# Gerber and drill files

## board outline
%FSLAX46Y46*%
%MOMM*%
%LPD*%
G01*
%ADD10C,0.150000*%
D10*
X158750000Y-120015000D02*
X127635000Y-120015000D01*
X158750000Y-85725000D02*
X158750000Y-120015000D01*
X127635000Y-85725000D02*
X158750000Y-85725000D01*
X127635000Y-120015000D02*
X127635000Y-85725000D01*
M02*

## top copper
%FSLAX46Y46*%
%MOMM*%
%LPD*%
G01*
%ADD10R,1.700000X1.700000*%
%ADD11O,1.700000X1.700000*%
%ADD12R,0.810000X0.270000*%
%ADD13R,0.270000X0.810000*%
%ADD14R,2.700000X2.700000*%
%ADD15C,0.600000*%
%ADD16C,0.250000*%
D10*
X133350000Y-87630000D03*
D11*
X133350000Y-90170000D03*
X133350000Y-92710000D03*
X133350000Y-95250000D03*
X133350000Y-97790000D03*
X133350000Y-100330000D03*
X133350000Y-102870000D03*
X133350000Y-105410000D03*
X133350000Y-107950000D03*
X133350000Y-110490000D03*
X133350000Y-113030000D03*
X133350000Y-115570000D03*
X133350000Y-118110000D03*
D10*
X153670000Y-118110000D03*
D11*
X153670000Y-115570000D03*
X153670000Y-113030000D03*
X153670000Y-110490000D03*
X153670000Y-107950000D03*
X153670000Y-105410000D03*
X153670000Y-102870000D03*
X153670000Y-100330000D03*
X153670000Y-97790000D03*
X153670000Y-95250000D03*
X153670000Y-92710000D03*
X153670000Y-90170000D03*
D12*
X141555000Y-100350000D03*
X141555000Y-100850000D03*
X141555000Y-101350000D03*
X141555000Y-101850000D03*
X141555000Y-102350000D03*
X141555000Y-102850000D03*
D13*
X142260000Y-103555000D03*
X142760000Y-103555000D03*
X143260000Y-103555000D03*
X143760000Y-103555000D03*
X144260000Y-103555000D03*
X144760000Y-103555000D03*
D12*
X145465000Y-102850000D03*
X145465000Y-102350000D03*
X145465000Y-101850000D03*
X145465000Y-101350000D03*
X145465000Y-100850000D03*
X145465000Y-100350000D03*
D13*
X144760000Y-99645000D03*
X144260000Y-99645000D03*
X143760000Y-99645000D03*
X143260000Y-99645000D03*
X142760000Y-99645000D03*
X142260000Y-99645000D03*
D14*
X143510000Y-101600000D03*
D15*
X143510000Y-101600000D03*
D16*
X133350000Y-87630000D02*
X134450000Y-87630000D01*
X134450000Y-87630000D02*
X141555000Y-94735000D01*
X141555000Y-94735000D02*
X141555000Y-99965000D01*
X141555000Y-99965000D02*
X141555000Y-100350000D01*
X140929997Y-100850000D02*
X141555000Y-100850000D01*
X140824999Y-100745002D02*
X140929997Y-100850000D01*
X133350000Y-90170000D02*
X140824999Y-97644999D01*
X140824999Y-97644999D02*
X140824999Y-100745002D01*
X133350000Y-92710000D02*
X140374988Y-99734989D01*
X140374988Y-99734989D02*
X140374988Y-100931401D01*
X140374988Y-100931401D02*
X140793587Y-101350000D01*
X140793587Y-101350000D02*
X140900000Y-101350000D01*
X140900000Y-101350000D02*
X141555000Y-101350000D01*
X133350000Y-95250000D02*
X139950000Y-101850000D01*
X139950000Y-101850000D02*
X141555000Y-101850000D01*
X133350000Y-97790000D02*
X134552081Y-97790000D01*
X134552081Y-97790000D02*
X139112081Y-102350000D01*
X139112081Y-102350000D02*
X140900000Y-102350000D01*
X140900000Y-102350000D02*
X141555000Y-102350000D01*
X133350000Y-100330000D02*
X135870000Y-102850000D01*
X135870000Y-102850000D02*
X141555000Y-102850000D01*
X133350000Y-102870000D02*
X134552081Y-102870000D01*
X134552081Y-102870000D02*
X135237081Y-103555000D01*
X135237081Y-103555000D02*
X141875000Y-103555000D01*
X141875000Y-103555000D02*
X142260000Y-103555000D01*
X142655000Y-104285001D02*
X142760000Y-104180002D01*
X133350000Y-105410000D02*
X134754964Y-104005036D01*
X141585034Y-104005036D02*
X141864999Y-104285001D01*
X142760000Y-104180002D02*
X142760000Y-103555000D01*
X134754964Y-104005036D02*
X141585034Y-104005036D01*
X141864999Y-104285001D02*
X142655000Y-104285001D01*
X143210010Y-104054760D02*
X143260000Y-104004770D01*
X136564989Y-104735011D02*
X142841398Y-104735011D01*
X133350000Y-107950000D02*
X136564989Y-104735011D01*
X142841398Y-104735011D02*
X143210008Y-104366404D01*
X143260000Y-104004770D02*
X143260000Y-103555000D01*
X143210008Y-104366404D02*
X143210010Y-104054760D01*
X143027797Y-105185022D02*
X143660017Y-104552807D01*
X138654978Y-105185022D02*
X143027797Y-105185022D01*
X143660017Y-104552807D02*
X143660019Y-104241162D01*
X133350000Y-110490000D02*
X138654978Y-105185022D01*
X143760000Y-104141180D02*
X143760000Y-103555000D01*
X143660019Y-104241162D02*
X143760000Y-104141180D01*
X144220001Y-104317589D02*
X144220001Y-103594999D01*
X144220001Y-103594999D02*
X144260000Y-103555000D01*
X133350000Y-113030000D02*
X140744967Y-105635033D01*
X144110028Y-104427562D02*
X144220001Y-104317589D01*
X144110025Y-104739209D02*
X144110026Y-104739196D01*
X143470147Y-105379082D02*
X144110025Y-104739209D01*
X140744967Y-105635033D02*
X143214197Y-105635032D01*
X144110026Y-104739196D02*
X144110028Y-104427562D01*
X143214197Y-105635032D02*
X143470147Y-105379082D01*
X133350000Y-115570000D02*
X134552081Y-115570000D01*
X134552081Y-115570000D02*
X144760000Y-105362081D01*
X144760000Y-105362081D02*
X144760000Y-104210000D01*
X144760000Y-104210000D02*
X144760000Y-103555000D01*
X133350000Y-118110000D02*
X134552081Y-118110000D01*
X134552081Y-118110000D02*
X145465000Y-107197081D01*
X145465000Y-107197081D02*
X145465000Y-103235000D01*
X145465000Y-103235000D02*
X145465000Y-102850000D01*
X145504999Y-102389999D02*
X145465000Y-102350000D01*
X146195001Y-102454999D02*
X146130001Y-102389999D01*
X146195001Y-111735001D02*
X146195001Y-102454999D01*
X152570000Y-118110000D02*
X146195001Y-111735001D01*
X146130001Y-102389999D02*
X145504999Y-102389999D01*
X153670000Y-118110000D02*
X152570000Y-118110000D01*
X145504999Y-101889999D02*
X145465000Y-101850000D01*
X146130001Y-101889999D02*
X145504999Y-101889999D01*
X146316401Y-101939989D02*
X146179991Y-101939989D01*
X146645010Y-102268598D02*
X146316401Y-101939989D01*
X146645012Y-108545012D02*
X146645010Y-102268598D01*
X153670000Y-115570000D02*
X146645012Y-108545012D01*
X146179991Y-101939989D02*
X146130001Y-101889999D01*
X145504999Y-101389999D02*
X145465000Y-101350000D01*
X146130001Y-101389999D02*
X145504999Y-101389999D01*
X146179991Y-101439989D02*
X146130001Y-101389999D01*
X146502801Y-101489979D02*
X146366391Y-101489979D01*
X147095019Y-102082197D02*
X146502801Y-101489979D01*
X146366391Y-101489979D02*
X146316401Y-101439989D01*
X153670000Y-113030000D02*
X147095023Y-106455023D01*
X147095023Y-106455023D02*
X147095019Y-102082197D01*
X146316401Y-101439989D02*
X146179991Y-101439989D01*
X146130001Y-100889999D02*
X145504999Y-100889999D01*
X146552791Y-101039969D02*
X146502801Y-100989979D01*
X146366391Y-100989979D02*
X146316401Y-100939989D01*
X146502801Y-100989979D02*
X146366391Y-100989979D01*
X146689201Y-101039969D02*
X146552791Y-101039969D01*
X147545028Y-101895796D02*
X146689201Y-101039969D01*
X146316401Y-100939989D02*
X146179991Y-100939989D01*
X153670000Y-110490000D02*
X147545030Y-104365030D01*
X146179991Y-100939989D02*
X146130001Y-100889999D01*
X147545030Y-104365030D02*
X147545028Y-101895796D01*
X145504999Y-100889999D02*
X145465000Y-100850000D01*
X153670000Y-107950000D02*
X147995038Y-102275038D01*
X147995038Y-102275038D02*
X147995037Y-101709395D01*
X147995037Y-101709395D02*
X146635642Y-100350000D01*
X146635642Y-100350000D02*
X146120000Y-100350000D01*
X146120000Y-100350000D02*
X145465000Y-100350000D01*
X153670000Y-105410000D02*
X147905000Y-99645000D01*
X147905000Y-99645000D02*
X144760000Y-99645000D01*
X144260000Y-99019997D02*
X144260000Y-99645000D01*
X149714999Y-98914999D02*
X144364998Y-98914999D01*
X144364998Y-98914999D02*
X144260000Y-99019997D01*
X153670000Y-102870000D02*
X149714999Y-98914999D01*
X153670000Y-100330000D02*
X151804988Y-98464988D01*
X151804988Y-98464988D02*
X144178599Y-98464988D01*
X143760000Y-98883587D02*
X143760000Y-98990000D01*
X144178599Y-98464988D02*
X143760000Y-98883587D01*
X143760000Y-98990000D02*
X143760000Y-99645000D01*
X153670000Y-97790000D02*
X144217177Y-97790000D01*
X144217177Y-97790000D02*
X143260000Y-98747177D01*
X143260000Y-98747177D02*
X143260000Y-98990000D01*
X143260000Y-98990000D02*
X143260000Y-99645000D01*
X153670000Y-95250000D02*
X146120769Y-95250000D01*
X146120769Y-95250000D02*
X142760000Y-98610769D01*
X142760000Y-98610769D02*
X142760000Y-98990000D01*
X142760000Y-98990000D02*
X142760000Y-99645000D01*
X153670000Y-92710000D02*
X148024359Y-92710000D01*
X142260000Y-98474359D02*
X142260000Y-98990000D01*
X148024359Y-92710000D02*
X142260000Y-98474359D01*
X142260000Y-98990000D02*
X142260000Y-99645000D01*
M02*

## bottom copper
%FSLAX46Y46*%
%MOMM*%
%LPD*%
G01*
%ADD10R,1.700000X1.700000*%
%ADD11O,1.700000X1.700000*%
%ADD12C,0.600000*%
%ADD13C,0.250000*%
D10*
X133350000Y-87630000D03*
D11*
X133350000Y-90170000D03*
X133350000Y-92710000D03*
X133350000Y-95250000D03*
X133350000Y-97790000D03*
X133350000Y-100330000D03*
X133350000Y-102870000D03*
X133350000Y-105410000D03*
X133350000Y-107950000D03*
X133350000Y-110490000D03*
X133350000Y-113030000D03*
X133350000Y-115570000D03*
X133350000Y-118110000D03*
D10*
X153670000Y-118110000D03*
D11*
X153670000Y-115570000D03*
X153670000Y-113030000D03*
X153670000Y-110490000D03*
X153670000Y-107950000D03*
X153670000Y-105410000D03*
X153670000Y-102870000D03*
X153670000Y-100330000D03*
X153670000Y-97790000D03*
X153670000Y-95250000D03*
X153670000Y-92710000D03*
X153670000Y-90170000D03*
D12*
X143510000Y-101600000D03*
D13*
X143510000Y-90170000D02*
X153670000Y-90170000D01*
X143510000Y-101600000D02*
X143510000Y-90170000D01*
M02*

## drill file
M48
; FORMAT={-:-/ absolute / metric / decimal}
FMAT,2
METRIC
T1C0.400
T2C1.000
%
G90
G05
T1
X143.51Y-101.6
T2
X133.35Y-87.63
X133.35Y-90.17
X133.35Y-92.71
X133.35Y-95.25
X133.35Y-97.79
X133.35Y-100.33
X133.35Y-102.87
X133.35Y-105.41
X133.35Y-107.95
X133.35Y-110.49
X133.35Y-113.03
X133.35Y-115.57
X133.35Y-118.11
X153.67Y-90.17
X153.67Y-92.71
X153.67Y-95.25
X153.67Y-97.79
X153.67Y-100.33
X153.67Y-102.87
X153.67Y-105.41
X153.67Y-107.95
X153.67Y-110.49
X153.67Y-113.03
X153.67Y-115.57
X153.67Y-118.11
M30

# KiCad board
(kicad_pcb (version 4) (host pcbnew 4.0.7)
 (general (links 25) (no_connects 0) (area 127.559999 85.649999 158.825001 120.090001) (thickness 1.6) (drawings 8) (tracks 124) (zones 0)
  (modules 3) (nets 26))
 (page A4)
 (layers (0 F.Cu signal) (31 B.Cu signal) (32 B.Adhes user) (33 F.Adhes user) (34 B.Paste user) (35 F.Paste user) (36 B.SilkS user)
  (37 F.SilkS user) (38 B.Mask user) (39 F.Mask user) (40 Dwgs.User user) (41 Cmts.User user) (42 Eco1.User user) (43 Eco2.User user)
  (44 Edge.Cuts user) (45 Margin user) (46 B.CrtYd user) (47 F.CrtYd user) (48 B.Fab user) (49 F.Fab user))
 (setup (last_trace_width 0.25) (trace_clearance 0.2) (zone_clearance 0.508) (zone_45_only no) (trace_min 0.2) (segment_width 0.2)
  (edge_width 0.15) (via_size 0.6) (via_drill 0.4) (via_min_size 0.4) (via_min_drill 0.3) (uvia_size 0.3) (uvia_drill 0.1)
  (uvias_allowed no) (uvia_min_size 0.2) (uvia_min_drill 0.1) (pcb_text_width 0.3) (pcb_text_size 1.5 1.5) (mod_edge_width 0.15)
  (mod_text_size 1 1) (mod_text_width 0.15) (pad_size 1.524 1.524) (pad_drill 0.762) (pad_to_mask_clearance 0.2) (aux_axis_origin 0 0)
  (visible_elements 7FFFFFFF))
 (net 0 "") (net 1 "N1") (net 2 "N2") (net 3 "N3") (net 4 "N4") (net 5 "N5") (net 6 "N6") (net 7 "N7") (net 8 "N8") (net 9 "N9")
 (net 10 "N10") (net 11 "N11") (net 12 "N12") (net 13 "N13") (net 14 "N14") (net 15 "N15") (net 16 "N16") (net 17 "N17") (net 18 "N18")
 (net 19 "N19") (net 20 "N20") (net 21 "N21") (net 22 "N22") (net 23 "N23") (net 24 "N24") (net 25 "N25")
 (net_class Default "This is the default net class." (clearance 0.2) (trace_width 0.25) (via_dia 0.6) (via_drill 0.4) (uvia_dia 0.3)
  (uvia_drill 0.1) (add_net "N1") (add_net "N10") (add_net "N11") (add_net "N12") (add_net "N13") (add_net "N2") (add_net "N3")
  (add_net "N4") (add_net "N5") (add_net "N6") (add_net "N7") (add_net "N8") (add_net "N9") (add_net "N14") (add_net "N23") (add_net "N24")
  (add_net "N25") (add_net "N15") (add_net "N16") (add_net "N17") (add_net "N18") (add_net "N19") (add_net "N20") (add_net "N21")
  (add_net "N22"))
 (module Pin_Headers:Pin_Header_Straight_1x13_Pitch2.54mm (layer F.Cu) (at 133.35 87.63)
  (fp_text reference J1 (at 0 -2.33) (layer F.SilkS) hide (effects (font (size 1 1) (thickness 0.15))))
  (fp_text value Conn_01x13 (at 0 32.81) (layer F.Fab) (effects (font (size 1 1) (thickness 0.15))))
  (pad 1 thru_hole rect (at 0 0) (size 1.7 1.7) (drill 1) (layers *.Cu *.Mask) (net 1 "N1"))
  (pad 2 thru_hole oval (at 0 2.54) (size 1.7 1.7) (drill 1) (layers *.Cu *.Mask) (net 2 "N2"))
  (pad 3 thru_hole oval (at 0 5.08) (size 1.7 1.7) (drill 1) (layers *.Cu *.Mask) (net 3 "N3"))
  (pad 4 thru_hole oval (at 0 7.62) (size 1.7 1.7) (drill 1) (layers *.Cu *.Mask) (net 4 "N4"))
  (pad 5 thru_hole oval (at 0 10.16) (size 1.7 1.7) (drill 1) (layers *.Cu *.Mask) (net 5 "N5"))
  (pad 6 thru_hole oval (at 0 12.7) (size 1.7 1.7) (drill 1) (layers *.Cu *.Mask) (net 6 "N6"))
  (pad 7 thru_hole oval (at 0 15.24) (size 1.7 1.7) (drill 1) (layers *.Cu *.Mask) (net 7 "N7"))
  (pad 8 thru_hole oval (at 0 17.78) (size 1.7 1.7) (drill 1) (layers *.Cu *.Mask) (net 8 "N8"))
  (pad 9 thru_hole oval (at 0 20.32) (size 1.7 1.7) (drill 1) (layers *.Cu *.Mask) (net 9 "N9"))
  (pad 10 thru_hole oval (at 0 22.86) (size 1.7 1.7) (drill 1) (layers *.Cu *.Mask) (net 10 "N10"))
  (pad 11 thru_hole oval (at 0 25.4) (size 1.7 1.7) (drill 1) (layers *.Cu *.Mask) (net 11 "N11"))
  (pad 12 thru_hole oval (at 0 27.94) (size 1.7 1.7) (drill 1) (layers *.Cu *.Mask) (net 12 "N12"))
  (pad 13 thru_hole oval (at 0 30.48) (size 1.7 1.7) (drill 1) (layers *.Cu *.Mask) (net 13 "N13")))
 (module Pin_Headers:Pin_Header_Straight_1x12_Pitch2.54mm (layer F.Cu) (at 153.67 118.11 180)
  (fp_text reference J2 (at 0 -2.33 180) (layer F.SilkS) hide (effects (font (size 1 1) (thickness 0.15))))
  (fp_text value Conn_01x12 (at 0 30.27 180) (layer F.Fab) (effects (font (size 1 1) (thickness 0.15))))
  (pad 1 thru_hole rect (at 0 0 180) (size 1.7 1.7) (drill 1) (layers *.Cu *.Mask) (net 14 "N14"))
  (pad 2 thru_hole oval (at 0 2.54 180) (size 1.7 1.7) (drill 1) (layers *.Cu *.Mask) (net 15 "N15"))
  (pad 3 thru_hole oval (at 0 5.08 180) (size 1.7 1.7) (drill 1) (layers *.Cu *.Mask) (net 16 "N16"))
  (pad 4 thru_hole oval (at 0 7.62 180) (size 1.7 1.7) (drill 1) (layers *.Cu *.Mask) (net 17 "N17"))
  (pad 5 thru_hole oval (at 0 10.16 180) (size 1.7 1.7) (drill 1) (layers *.Cu *.Mask) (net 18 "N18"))
  (pad 6 thru_hole oval (at 0 12.7 180) (size 1.7 1.7) (drill 1) (layers *.Cu *.Mask) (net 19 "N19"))
  (pad 7 thru_hole oval (at 0 15.24 180) (size 1.7 1.7) (drill 1) (layers *.Cu *.Mask) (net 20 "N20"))
  (pad 8 thru_hole oval (at 0 17.78 180) (size 1.7 1.7) (drill 1) (layers *.Cu *.Mask) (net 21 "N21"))
  (pad 9 thru_hole oval (at 0 20.32 180) (size 1.7 1.7) (drill 1) (layers *.Cu *.Mask) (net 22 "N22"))
  (pad 10 thru_hole oval (at 0 22.86 180) (size 1.7 1.7) (drill 1) (layers *.Cu *.Mask) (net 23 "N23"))
  (pad 11 thru_hole oval (at 0 25.4 180) (size 1.7 1.7) (drill 1) (layers *.Cu *.Mask) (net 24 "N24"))
  (pad 12 thru_hole oval (at 0 27.94 180) (size 1.7 1.7) (drill 1) (layers *.Cu *.Mask) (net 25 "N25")))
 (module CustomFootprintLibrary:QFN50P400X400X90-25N (layer F.Cu) (at 143.51 101.6)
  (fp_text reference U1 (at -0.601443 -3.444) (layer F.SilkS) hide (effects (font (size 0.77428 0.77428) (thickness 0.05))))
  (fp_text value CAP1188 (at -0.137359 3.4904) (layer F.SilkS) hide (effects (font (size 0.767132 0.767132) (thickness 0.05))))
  (pad 1 smd rect (at -1.955 -1.25) (size 0.81 0.27) (layers F.Cu F.Paste F.Mask) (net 1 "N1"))
  (pad 2 smd rect (at -1.955 -0.75) (size 0.81 0.27) (layers F.Cu F.Paste F.Mask) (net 2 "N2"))
  (pad 3 smd rect (at -1.955 -0.25) (size 0.81 0.27) (layers F.Cu F.Paste F.Mask) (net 3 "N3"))
  (pad 4 smd rect (at -1.955 0.25) (size 0.81 0.27) (layers F.Cu F.Paste F.Mask) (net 4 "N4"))
  (pad 5 smd rect (at -1.955 0.75) (size 0.81 0.27) (layers F.Cu F.Paste F.Mask) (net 5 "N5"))
  (pad 6 smd rect (at -1.955 1.25) (size 0.81 0.27) (layers F.Cu F.Paste F.Mask) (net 6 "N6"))
  (pad 7 smd rect (at -1.25 1.955 90) (size 0.81 0.27) (layers F.Cu F.Paste F.Mask) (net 7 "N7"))
  (pad 8 smd rect (at -0.75 1.955 90) (size 0.81 0.27) (layers F.Cu F.Paste F.Mask) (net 8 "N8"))
  (pad 9 smd rect (at -0.25 1.955 90) (size 0.81 0.27) (layers F.Cu F.Paste F.Mask) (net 9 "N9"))
  (pad 10 smd rect (at 0.25 1.955 90) (size 0.81 0.27) (layers F.Cu F.Paste F.Mask) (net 10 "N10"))
  (pad 11 smd rect (at 0.75 1.955 90) (size 0.81 0.27) (layers F.Cu F.Paste F.Mask) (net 11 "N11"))
  (pad 12 smd rect (at 1.25 1.955 90) (size 0.81 0.27) (layers F.Cu F.Paste F.Mask) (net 12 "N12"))
  (pad 13 smd rect (at 1.955 1.25 180) (size 0.81 0.27) (layers F.Cu F.Paste F.Mask) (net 13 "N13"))
  (pad 14 smd rect (at 1.955 0.75 180) (size 0.81 0.27) (layers F.Cu F.Paste F.Mask) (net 14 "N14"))
  (pad 15 smd rect (at 1.955 0.25 180) (size 0.81 0.27) (layers F.Cu F.Paste F.Mask) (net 15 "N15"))
  (pad 16 smd rect (at 1.955 -0.25 180) (size 0.81 0.27) (layers F.Cu F.Paste F.Mask) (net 16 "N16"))
  (pad 17 smd rect (at 1.955 -0.75 180) (size 0.81 0.27) (layers F.Cu F.Paste F.Mask) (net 17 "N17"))
  (pad 18 smd rect (at 1.955 -1.25 180) (size 0.81 0.27) (layers F.Cu F.Paste F.Mask) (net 18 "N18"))
  (pad 19 smd rect (at 1.25 -1.955 270) (size 0.81 0.27) (layers F.Cu F.Paste F.Mask) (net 19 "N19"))
  (pad 20 smd rect (at 0.75 -1.955 270) (size 0.81 0.27) (layers F.Cu F.Paste F.Mask) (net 20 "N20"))
  (pad 21 smd rect (at 0.25 -1.955 270) (size 0.81 0.27) (layers F.Cu F.Paste F.Mask) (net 21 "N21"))
  (pad 22 smd rect (at -0.25 -1.955 270) (size 0.81 0.27) (layers F.Cu F.Paste F.Mask) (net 22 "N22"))
  (pad 23 smd rect (at -0.75 -1.955 270) (size 0.81 0.27) (layers F.Cu F.Paste F.Mask) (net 23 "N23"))
  (pad 24 smd rect (at -1.25 -1.955 270) (size 0.81 0.27) (layers F.Cu F.Paste F.Mask) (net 24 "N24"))
  (pad 25 smd rect (at 0 0 270) (size 2.7 2.7) (layers F.Cu F.Paste F.Mask) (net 25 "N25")))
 (gr_line (start 158.75 120.015) (end 127.635 120.015) (layer Edge.Cuts) (width 0.15))
 (gr_line (start 158.75 85.725) (end 158.75 120.015) (layer Edge.Cuts) (width 0.15))
 (gr_line (start 127.635 85.725) (end 158.75 85.725) (layer Edge.Cuts) (width 0.15))
 (gr_line (start 127.635 120.015) (end 127.635 85.725) (layer Edge.Cuts) (width 0.15))
 (segment (start 133.35 87.63) (end 134.45 87.63) (width 0.25) (layer F.Cu) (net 1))
 (segment (start 134.45 87.63) (end 141.555 94.735) (width 0.25) (layer F.Cu) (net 1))
 (segment (start 141.555 94.735) (end 141.555 99.965) (width 0.25) (layer F.Cu) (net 1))
 (segment (start 141.555 99.965) (end 141.555 100.35) (width 0.25) (layer F.Cu) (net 1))
 (segment (start 140.929997 100.85) (end 141.555 100.85) (width 0.25) (layer F.Cu) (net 2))
 (segment (start 140.824999 100.745002) (end 140.929997 100.85) (width 0.25) (layer F.Cu) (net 2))
 (segment (start 133.35 90.17) (end 140.824999 97.644999) (width 0.25) (layer F.Cu) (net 2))
 (segment (start 140.824999 97.644999) (end 140.824999 100.745002) (width 0.25) (layer F.Cu) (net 2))
 (segment (start 133.35 92.71) (end 140.374988 99.734989) (width 0.25) (layer F.Cu) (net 3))
 (segment (start 140.374988 99.734989) (end 140.374988 100.931401) (width 0.25) (layer F.Cu) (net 3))
 (segment (start 140.374988 100.931401) (end 140.793587 101.35) (width 0.25) (layer F.Cu) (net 3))
 (segment (start 140.793587 101.35) (end 140.9 101.35) (width 0.25) (layer F.Cu) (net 3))
 (segment (start 140.9 101.35) (end 141.555 101.35) (width 0.25) (layer F.Cu) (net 3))
 (segment (start 133.35 95.25) (end 139.95 101.85) (width 0.25) (layer F.Cu) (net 4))
 (segment (start 139.95 101.85) (end 141.555 101.85) (width 0.25) (layer F.Cu) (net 4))
 (segment (start 133.35 97.79) (end 134.552081 97.79) (width 0.25) (layer F.Cu) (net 5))
 (segment (start 134.552081 97.79) (end 139.112081 102.35) (width 0.25) (layer F.Cu) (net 5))
 (segment (start 139.112081 102.35) (end 140.9 102.35) (width 0.25) (layer F.Cu) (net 5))
 (segment (start 140.9 102.35) (end 141.555 102.35) (width 0.25) (layer F.Cu) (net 5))
 (segment (start 133.35 100.33) (end 135.87 102.85) (width 0.25) (layer F.Cu) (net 6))
 (segment (start 135.87 102.85) (end 141.555 102.85) (width 0.25) (layer F.Cu) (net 6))
 (segment (start 133.35 102.87) (end 134.552081 102.87) (width 0.25) (layer F.Cu) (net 7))
 (segment (start 134.552081 102.87) (end 135.237081 103.555) (width 0.25) (layer F.Cu) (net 7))
 (segment (start 135.237081 103.555) (end 141.875 103.555) (width 0.25) (layer F.Cu) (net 7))
 (segment (start 141.875 103.555) (end 142.26 103.555) (width 0.25) (layer F.Cu) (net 7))
 (segment (start 142.655 104.285001) (end 142.76 104.180002) (width 0.25) (layer F.Cu) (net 8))
 (segment (start 133.35 105.41) (end 134.754964 104.005036) (width 0.25) (layer F.Cu) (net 8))
 (segment (start 141.585034 104.005036) (end 141.864999 104.285001) (width 0.25) (layer F.Cu) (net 8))
 (segment (start 142.76 104.180002) (end 142.76 103.555) (width 0.25) (layer F.Cu) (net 8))
 (segment (start 134.754964 104.005036) (end 141.585034 104.005036) (width 0.25) (layer F.Cu) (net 8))
 (segment (start 141.864999 104.285001) (end 142.655 104.285001) (width 0.25) (layer F.Cu) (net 8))
 (segment (start 143.21001 104.05476) (end 143.26 104.00477) (width 0.25) (layer F.Cu) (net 9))
 (segment (start 136.564989 104.735011) (end 142.841398 104.735011) (width 0.25) (layer F.Cu) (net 9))
 (segment (start 133.35 107.95) (end 136.564989 104.735011) (width 0.25) (layer F.Cu) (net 9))
 (segment (start 142.841398 104.735011) (end 143.210008 104.366404) (width 0.25) (layer F.Cu) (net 9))
 (segment (start 143.26 104.00477) (end 143.26 103.555) (width 0.25) (layer F.Cu) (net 9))
 (segment (start 143.210008 104.366404) (end 143.21001 104.05476) (width 0.25) (layer F.Cu) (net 9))
 (segment (start 143.027797 105.185022) (end 143.660017 104.552807) (width 0.25) (layer F.Cu) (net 10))
 (segment (start 138.654978 105.185022) (end 143.027797 105.185022) (width 0.25) (layer F.Cu) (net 10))
 (segment (start 143.660017 104.552807) (end 143.660019 104.241162) (width 0.25) (layer F.Cu) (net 10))
 (segment (start 133.35 110.49) (end 138.654978 105.185022) (width 0.25) (layer F.Cu) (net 10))
 (segment (start 143.76 104.14118) (end 143.76 103.555) (width 0.25) (layer F.Cu) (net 10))
 (segment (start 143.660019 104.241162) (end 143.76 104.14118) (width 0.25) (layer F.Cu) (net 10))
 (segment (start 144.220001 104.317589) (end 144.220001 103.594999) (width 0.25) (layer F.Cu) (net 11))
 (segment (start 144.220001 103.594999) (end 144.26 103.555) (width 0.25) (layer F.Cu) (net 11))
 (segment (start 133.35 113.03) (end 140.744967 105.635033) (width 0.25) (layer F.Cu) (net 11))
 (segment (start 144.110028 104.427562) (end 144.220001 104.317589) (width 0.25) (layer F.Cu) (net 11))
 (segment (start 144.110025 104.739209) (end 144.110026 104.739196) (width 0.25) (layer F.Cu) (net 11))
 (segment (start 143.470147 105.379082) (end 144.110025 104.739209) (width 0.25) (layer F.Cu) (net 11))
 (segment (start 140.744967 105.635033) (end 143.214197 105.635032) (width 0.25) (layer F.Cu) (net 11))
 (segment (start 144.110026 104.739196) (end 144.110028 104.427562) (width 0.25) (layer F.Cu) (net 11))
 (segment (start 143.214197 105.635032) (end 143.470147 105.379082) (width 0.25) (layer F.Cu) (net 11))
 (segment (start 133.35 115.57) (end 134.552081 115.57) (width 0.25) (layer F.Cu) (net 12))
 (segment (start 134.552081 115.57) (end 144.76 105.362081) (width 0.25) (layer F.Cu) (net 12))
 (segment (start 144.76 105.362081) (end 144.76 104.21) (width 0.25) (layer F.Cu) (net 12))
 (segment (start 144.76 104.21) (end 144.76 103.555) (width 0.25) (layer F.Cu) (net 12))
 (segment (start 133.35 118.11) (end 134.552081 118.11) (width 0.25) (layer F.Cu) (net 13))
 (segment (start 134.552081 118.11) (end 145.465 107.197081) (width 0.25) (layer F.Cu) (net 13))
 (segment (start 145.465 107.197081) (end 145.465 103.235) (width 0.25) (layer F.Cu) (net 13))
 (segment (start 145.465 103.235) (end 145.465 102.85) (width 0.25) (layer F.Cu) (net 13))
 (segment (start 145.504999 102.389999) (end 145.465 102.35) (width 0.25) (layer F.Cu) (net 14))
 (segment (start 146.195001 102.454999) (end 146.130001 102.389999) (width 0.25) (layer F.Cu) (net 14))
 (segment (start 146.195001 111.735001) (end 146.195001 102.454999) (width 0.25) (layer F.Cu) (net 14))
 (segment (start 152.57 118.11) (end 146.195001 111.735001) (width 0.25) (layer F.Cu) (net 14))
 (segment (start 146.130001 102.389999) (end 145.504999 102.389999) (width 0.25) (layer F.Cu) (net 14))
 (segment (start 153.67 118.11) (end 152.57 118.11) (width 0.25) (layer F.Cu) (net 14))
 (segment (start 145.504999 101.889999) (end 145.465 101.85) (width 0.25) (layer F.Cu) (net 15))
 (segment (start 146.130001 101.889999) (end 145.504999 101.889999) (width 0.25) (layer F.Cu) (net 15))
 (segment (start 146.316401 101.939989) (end 146.179991 101.939989) (width 0.25) (layer F.Cu) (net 15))
 (segment (start 146.64501 102.268598) (end 146.316401 101.939989) (width 0.25) (layer F.Cu) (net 15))
 (segment (start 146.645012 108.545012) (end 146.64501 102.268598) (width 0.25) (layer F.Cu) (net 15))
 (segment (start 153.67 115.57) (end 146.645012 108.545012) (width 0.25) (layer F.Cu) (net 15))
 (segment (start 146.179991 101.939989) (end 146.130001 101.889999) (width 0.25) (layer F.Cu) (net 15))
 (segment (start 145.504999 101.389999) (end 145.465 101.35) (width 0.25) (layer F.Cu) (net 16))
 (segment (start 146.130001 101.389999) (end 145.504999 101.389999) (width 0.25) (layer F.Cu) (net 16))
 (segment (start 146.179991 101.439989) (end 146.130001 101.389999) (width 0.25) (layer F.Cu) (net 16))
 (segment (start 146.502801 101.489979) (end 146.366391 101.489979) (width 0.25) (layer F.Cu) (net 16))
 (segment (start 147.095019 102.082197) (end 146.502801 101.489979) (width 0.25) (layer F.Cu) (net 16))
 (segment (start 146.366391 101.489979) (end 146.316401 101.439989) (width 0.25) (layer F.Cu) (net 16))
 (segment (start 153.67 113.03) (end 147.095023 106.455023) (width 0.25) (layer F.Cu) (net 16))
 (segment (start 147.095023 106.455023) (end 147.095019 102.082197) (width 0.25) (layer F.Cu) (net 16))
 (segment (start 146.316401 101.439989) (end 146.179991 101.439989) (width 0.25) (layer F.Cu) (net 16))
 (segment (start 146.130001 100.889999) (end 145.504999 100.889999) (width 0.25) (layer F.Cu) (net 17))
 (segment (start 146.552791 101.039969) (end 146.502801 100.989979) (width 0.25) (layer F.Cu) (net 17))
 (segment (start 146.366391 100.989979) (end 146.316401 100.939989) (width 0.25) (layer F.Cu) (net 17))
 (segment (start 146.502801 100.989979) (end 146.366391 100.989979) (width 0.25) (layer F.Cu) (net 17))
 (segment (start 146.689201 101.039969) (end 146.552791 101.039969) (width 0.25) (layer F.Cu) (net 17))
 (segment (start 147.545028 101.895796) (end 146.689201 101.039969) (width 0.25) (layer F.Cu) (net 17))
 (segment (start 146.316401 100.939989) (end 146.179991 100.939989) (width 0.25) (layer F.Cu) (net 17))
 (segment (start 153.67 110.49) (end 147.54503 104.36503) (width 0.25) (layer F.Cu) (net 17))
 (segment (start 146.179991 100.939989) (end 146.130001 100.889999) (width 0.25) (layer F.Cu) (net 17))
 (segment (start 147.54503 104.36503) (end 147.545028 101.895796) (width 0.25) (layer F.Cu) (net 17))
 (segment (start 145.504999 100.889999) (end 145.465 100.85) (width 0.25) (layer F.Cu) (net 17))
 (segment (start 153.67 107.95) (end 147.995038 102.275038) (width 0.25) (layer F.Cu) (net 18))
 (segment (start 147.995038 102.275038) (end 147.995037 101.709395) (width 0.25) (layer F.Cu) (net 18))
 (segment (start 147.995037 101.709395) (end 146.635642 100.35) (width 0.25) (layer F.Cu) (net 18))
 (segment (start 146.635642 100.35) (end 146.12 100.35) (width 0.25) (layer F.Cu) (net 18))
 (segment (start 146.12 100.35) (end 145.465 100.35) (width 0.25) (layer F.Cu) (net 18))
 (segment (start 153.67 105.41) (end 147.905 99.645) (width 0.25) (layer F.Cu) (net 19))
 (segment (start 147.905 99.645) (end 144.76 99.645) (width 0.25) (layer F.Cu) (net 19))
 (segment (start 144.26 99.019997) (end 144.26 99.645) (width 0.25) (layer F.Cu) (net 20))
 (segment (start 149.714999 98.914999) (end 144.364998 98.914999) (width 0.25) (layer F.Cu) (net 20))
 (segment (start 144.364998 98.914999) (end 144.26 99.019997) (width 0.25) (layer F.Cu) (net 20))
 (segment (start 153.67 102.87) (end 149.714999 98.914999) (width 0.25) (layer F.Cu) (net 20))
 (segment (start 153.67 100.33) (end 151.804988 98.464988) (width 0.25) (layer F.Cu) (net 21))
 (segment (start 151.804988 98.464988) (end 144.178599 98.464988) (width 0.25) (layer F.Cu) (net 21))
 (segment (start 143.76 98.883587) (end 143.76 98.99) (width 0.25) (layer F.Cu) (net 21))
 (segment (start 144.178599 98.464988) (end 143.76 98.883587) (width 0.25) (layer F.Cu) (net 21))
 (segment (start 143.76 98.99) (end 143.76 99.645) (width 0.25) (layer F.Cu) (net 21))
 (segment (start 153.67 97.79) (end 144.217177 97.79) (width 0.25) (layer F.Cu) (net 22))
 (segment (start 144.217177 97.79) (end 143.26 98.747177) (width 0.25) (layer F.Cu) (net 22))
 (segment (start 143.26 98.747177) (end 143.26 98.99) (width 0.25) (layer F.Cu) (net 22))
 (segment (start 143.26 98.99) (end 143.26 99.645) (width 0.25) (layer F.Cu) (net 22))
 (segment (start 153.67 95.25) (end 146.120769 95.25) (width 0.25) (layer F.Cu) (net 23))
 (segment (start 146.120769 95.25) (end 142.76 98.610769) (width 0.25) (layer F.Cu) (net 23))
 (segment (start 142.76 98.610769) (end 142.76 98.99) (width 0.25) (layer F.Cu) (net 23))
 (segment (start 142.76 98.99) (end 142.76 99.645) (width 0.25) (layer F.Cu) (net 23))
 (segment (start 153.67 92.71) (end 148.024359 92.71) (width 0.25) (layer F.Cu) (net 24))
 (segment (start 142.26 98.474359) (end 142.26 98.99) (width 0.25) (layer F.Cu) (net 24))
 (segment (start 148.024359 92.71) (end 142.26 98.474359) (width 0.25) (layer F.Cu) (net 24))
 (segment (start 142.26 98.99) (end 142.26 99.645) (width 0.25) (layer F.Cu) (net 24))
 (segment (start 143.51 90.17) (end 153.67 90.17) (width 0.25) (layer B.Cu) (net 25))
 (segment (start 143.51 101.6) (end 143.51 90.17) (width 0.25) (layer B.Cu) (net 25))
 (via (at 143.51 101.6) (size 0.6) (drill 0.4) (layers F.Cu B.Cu) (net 25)))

